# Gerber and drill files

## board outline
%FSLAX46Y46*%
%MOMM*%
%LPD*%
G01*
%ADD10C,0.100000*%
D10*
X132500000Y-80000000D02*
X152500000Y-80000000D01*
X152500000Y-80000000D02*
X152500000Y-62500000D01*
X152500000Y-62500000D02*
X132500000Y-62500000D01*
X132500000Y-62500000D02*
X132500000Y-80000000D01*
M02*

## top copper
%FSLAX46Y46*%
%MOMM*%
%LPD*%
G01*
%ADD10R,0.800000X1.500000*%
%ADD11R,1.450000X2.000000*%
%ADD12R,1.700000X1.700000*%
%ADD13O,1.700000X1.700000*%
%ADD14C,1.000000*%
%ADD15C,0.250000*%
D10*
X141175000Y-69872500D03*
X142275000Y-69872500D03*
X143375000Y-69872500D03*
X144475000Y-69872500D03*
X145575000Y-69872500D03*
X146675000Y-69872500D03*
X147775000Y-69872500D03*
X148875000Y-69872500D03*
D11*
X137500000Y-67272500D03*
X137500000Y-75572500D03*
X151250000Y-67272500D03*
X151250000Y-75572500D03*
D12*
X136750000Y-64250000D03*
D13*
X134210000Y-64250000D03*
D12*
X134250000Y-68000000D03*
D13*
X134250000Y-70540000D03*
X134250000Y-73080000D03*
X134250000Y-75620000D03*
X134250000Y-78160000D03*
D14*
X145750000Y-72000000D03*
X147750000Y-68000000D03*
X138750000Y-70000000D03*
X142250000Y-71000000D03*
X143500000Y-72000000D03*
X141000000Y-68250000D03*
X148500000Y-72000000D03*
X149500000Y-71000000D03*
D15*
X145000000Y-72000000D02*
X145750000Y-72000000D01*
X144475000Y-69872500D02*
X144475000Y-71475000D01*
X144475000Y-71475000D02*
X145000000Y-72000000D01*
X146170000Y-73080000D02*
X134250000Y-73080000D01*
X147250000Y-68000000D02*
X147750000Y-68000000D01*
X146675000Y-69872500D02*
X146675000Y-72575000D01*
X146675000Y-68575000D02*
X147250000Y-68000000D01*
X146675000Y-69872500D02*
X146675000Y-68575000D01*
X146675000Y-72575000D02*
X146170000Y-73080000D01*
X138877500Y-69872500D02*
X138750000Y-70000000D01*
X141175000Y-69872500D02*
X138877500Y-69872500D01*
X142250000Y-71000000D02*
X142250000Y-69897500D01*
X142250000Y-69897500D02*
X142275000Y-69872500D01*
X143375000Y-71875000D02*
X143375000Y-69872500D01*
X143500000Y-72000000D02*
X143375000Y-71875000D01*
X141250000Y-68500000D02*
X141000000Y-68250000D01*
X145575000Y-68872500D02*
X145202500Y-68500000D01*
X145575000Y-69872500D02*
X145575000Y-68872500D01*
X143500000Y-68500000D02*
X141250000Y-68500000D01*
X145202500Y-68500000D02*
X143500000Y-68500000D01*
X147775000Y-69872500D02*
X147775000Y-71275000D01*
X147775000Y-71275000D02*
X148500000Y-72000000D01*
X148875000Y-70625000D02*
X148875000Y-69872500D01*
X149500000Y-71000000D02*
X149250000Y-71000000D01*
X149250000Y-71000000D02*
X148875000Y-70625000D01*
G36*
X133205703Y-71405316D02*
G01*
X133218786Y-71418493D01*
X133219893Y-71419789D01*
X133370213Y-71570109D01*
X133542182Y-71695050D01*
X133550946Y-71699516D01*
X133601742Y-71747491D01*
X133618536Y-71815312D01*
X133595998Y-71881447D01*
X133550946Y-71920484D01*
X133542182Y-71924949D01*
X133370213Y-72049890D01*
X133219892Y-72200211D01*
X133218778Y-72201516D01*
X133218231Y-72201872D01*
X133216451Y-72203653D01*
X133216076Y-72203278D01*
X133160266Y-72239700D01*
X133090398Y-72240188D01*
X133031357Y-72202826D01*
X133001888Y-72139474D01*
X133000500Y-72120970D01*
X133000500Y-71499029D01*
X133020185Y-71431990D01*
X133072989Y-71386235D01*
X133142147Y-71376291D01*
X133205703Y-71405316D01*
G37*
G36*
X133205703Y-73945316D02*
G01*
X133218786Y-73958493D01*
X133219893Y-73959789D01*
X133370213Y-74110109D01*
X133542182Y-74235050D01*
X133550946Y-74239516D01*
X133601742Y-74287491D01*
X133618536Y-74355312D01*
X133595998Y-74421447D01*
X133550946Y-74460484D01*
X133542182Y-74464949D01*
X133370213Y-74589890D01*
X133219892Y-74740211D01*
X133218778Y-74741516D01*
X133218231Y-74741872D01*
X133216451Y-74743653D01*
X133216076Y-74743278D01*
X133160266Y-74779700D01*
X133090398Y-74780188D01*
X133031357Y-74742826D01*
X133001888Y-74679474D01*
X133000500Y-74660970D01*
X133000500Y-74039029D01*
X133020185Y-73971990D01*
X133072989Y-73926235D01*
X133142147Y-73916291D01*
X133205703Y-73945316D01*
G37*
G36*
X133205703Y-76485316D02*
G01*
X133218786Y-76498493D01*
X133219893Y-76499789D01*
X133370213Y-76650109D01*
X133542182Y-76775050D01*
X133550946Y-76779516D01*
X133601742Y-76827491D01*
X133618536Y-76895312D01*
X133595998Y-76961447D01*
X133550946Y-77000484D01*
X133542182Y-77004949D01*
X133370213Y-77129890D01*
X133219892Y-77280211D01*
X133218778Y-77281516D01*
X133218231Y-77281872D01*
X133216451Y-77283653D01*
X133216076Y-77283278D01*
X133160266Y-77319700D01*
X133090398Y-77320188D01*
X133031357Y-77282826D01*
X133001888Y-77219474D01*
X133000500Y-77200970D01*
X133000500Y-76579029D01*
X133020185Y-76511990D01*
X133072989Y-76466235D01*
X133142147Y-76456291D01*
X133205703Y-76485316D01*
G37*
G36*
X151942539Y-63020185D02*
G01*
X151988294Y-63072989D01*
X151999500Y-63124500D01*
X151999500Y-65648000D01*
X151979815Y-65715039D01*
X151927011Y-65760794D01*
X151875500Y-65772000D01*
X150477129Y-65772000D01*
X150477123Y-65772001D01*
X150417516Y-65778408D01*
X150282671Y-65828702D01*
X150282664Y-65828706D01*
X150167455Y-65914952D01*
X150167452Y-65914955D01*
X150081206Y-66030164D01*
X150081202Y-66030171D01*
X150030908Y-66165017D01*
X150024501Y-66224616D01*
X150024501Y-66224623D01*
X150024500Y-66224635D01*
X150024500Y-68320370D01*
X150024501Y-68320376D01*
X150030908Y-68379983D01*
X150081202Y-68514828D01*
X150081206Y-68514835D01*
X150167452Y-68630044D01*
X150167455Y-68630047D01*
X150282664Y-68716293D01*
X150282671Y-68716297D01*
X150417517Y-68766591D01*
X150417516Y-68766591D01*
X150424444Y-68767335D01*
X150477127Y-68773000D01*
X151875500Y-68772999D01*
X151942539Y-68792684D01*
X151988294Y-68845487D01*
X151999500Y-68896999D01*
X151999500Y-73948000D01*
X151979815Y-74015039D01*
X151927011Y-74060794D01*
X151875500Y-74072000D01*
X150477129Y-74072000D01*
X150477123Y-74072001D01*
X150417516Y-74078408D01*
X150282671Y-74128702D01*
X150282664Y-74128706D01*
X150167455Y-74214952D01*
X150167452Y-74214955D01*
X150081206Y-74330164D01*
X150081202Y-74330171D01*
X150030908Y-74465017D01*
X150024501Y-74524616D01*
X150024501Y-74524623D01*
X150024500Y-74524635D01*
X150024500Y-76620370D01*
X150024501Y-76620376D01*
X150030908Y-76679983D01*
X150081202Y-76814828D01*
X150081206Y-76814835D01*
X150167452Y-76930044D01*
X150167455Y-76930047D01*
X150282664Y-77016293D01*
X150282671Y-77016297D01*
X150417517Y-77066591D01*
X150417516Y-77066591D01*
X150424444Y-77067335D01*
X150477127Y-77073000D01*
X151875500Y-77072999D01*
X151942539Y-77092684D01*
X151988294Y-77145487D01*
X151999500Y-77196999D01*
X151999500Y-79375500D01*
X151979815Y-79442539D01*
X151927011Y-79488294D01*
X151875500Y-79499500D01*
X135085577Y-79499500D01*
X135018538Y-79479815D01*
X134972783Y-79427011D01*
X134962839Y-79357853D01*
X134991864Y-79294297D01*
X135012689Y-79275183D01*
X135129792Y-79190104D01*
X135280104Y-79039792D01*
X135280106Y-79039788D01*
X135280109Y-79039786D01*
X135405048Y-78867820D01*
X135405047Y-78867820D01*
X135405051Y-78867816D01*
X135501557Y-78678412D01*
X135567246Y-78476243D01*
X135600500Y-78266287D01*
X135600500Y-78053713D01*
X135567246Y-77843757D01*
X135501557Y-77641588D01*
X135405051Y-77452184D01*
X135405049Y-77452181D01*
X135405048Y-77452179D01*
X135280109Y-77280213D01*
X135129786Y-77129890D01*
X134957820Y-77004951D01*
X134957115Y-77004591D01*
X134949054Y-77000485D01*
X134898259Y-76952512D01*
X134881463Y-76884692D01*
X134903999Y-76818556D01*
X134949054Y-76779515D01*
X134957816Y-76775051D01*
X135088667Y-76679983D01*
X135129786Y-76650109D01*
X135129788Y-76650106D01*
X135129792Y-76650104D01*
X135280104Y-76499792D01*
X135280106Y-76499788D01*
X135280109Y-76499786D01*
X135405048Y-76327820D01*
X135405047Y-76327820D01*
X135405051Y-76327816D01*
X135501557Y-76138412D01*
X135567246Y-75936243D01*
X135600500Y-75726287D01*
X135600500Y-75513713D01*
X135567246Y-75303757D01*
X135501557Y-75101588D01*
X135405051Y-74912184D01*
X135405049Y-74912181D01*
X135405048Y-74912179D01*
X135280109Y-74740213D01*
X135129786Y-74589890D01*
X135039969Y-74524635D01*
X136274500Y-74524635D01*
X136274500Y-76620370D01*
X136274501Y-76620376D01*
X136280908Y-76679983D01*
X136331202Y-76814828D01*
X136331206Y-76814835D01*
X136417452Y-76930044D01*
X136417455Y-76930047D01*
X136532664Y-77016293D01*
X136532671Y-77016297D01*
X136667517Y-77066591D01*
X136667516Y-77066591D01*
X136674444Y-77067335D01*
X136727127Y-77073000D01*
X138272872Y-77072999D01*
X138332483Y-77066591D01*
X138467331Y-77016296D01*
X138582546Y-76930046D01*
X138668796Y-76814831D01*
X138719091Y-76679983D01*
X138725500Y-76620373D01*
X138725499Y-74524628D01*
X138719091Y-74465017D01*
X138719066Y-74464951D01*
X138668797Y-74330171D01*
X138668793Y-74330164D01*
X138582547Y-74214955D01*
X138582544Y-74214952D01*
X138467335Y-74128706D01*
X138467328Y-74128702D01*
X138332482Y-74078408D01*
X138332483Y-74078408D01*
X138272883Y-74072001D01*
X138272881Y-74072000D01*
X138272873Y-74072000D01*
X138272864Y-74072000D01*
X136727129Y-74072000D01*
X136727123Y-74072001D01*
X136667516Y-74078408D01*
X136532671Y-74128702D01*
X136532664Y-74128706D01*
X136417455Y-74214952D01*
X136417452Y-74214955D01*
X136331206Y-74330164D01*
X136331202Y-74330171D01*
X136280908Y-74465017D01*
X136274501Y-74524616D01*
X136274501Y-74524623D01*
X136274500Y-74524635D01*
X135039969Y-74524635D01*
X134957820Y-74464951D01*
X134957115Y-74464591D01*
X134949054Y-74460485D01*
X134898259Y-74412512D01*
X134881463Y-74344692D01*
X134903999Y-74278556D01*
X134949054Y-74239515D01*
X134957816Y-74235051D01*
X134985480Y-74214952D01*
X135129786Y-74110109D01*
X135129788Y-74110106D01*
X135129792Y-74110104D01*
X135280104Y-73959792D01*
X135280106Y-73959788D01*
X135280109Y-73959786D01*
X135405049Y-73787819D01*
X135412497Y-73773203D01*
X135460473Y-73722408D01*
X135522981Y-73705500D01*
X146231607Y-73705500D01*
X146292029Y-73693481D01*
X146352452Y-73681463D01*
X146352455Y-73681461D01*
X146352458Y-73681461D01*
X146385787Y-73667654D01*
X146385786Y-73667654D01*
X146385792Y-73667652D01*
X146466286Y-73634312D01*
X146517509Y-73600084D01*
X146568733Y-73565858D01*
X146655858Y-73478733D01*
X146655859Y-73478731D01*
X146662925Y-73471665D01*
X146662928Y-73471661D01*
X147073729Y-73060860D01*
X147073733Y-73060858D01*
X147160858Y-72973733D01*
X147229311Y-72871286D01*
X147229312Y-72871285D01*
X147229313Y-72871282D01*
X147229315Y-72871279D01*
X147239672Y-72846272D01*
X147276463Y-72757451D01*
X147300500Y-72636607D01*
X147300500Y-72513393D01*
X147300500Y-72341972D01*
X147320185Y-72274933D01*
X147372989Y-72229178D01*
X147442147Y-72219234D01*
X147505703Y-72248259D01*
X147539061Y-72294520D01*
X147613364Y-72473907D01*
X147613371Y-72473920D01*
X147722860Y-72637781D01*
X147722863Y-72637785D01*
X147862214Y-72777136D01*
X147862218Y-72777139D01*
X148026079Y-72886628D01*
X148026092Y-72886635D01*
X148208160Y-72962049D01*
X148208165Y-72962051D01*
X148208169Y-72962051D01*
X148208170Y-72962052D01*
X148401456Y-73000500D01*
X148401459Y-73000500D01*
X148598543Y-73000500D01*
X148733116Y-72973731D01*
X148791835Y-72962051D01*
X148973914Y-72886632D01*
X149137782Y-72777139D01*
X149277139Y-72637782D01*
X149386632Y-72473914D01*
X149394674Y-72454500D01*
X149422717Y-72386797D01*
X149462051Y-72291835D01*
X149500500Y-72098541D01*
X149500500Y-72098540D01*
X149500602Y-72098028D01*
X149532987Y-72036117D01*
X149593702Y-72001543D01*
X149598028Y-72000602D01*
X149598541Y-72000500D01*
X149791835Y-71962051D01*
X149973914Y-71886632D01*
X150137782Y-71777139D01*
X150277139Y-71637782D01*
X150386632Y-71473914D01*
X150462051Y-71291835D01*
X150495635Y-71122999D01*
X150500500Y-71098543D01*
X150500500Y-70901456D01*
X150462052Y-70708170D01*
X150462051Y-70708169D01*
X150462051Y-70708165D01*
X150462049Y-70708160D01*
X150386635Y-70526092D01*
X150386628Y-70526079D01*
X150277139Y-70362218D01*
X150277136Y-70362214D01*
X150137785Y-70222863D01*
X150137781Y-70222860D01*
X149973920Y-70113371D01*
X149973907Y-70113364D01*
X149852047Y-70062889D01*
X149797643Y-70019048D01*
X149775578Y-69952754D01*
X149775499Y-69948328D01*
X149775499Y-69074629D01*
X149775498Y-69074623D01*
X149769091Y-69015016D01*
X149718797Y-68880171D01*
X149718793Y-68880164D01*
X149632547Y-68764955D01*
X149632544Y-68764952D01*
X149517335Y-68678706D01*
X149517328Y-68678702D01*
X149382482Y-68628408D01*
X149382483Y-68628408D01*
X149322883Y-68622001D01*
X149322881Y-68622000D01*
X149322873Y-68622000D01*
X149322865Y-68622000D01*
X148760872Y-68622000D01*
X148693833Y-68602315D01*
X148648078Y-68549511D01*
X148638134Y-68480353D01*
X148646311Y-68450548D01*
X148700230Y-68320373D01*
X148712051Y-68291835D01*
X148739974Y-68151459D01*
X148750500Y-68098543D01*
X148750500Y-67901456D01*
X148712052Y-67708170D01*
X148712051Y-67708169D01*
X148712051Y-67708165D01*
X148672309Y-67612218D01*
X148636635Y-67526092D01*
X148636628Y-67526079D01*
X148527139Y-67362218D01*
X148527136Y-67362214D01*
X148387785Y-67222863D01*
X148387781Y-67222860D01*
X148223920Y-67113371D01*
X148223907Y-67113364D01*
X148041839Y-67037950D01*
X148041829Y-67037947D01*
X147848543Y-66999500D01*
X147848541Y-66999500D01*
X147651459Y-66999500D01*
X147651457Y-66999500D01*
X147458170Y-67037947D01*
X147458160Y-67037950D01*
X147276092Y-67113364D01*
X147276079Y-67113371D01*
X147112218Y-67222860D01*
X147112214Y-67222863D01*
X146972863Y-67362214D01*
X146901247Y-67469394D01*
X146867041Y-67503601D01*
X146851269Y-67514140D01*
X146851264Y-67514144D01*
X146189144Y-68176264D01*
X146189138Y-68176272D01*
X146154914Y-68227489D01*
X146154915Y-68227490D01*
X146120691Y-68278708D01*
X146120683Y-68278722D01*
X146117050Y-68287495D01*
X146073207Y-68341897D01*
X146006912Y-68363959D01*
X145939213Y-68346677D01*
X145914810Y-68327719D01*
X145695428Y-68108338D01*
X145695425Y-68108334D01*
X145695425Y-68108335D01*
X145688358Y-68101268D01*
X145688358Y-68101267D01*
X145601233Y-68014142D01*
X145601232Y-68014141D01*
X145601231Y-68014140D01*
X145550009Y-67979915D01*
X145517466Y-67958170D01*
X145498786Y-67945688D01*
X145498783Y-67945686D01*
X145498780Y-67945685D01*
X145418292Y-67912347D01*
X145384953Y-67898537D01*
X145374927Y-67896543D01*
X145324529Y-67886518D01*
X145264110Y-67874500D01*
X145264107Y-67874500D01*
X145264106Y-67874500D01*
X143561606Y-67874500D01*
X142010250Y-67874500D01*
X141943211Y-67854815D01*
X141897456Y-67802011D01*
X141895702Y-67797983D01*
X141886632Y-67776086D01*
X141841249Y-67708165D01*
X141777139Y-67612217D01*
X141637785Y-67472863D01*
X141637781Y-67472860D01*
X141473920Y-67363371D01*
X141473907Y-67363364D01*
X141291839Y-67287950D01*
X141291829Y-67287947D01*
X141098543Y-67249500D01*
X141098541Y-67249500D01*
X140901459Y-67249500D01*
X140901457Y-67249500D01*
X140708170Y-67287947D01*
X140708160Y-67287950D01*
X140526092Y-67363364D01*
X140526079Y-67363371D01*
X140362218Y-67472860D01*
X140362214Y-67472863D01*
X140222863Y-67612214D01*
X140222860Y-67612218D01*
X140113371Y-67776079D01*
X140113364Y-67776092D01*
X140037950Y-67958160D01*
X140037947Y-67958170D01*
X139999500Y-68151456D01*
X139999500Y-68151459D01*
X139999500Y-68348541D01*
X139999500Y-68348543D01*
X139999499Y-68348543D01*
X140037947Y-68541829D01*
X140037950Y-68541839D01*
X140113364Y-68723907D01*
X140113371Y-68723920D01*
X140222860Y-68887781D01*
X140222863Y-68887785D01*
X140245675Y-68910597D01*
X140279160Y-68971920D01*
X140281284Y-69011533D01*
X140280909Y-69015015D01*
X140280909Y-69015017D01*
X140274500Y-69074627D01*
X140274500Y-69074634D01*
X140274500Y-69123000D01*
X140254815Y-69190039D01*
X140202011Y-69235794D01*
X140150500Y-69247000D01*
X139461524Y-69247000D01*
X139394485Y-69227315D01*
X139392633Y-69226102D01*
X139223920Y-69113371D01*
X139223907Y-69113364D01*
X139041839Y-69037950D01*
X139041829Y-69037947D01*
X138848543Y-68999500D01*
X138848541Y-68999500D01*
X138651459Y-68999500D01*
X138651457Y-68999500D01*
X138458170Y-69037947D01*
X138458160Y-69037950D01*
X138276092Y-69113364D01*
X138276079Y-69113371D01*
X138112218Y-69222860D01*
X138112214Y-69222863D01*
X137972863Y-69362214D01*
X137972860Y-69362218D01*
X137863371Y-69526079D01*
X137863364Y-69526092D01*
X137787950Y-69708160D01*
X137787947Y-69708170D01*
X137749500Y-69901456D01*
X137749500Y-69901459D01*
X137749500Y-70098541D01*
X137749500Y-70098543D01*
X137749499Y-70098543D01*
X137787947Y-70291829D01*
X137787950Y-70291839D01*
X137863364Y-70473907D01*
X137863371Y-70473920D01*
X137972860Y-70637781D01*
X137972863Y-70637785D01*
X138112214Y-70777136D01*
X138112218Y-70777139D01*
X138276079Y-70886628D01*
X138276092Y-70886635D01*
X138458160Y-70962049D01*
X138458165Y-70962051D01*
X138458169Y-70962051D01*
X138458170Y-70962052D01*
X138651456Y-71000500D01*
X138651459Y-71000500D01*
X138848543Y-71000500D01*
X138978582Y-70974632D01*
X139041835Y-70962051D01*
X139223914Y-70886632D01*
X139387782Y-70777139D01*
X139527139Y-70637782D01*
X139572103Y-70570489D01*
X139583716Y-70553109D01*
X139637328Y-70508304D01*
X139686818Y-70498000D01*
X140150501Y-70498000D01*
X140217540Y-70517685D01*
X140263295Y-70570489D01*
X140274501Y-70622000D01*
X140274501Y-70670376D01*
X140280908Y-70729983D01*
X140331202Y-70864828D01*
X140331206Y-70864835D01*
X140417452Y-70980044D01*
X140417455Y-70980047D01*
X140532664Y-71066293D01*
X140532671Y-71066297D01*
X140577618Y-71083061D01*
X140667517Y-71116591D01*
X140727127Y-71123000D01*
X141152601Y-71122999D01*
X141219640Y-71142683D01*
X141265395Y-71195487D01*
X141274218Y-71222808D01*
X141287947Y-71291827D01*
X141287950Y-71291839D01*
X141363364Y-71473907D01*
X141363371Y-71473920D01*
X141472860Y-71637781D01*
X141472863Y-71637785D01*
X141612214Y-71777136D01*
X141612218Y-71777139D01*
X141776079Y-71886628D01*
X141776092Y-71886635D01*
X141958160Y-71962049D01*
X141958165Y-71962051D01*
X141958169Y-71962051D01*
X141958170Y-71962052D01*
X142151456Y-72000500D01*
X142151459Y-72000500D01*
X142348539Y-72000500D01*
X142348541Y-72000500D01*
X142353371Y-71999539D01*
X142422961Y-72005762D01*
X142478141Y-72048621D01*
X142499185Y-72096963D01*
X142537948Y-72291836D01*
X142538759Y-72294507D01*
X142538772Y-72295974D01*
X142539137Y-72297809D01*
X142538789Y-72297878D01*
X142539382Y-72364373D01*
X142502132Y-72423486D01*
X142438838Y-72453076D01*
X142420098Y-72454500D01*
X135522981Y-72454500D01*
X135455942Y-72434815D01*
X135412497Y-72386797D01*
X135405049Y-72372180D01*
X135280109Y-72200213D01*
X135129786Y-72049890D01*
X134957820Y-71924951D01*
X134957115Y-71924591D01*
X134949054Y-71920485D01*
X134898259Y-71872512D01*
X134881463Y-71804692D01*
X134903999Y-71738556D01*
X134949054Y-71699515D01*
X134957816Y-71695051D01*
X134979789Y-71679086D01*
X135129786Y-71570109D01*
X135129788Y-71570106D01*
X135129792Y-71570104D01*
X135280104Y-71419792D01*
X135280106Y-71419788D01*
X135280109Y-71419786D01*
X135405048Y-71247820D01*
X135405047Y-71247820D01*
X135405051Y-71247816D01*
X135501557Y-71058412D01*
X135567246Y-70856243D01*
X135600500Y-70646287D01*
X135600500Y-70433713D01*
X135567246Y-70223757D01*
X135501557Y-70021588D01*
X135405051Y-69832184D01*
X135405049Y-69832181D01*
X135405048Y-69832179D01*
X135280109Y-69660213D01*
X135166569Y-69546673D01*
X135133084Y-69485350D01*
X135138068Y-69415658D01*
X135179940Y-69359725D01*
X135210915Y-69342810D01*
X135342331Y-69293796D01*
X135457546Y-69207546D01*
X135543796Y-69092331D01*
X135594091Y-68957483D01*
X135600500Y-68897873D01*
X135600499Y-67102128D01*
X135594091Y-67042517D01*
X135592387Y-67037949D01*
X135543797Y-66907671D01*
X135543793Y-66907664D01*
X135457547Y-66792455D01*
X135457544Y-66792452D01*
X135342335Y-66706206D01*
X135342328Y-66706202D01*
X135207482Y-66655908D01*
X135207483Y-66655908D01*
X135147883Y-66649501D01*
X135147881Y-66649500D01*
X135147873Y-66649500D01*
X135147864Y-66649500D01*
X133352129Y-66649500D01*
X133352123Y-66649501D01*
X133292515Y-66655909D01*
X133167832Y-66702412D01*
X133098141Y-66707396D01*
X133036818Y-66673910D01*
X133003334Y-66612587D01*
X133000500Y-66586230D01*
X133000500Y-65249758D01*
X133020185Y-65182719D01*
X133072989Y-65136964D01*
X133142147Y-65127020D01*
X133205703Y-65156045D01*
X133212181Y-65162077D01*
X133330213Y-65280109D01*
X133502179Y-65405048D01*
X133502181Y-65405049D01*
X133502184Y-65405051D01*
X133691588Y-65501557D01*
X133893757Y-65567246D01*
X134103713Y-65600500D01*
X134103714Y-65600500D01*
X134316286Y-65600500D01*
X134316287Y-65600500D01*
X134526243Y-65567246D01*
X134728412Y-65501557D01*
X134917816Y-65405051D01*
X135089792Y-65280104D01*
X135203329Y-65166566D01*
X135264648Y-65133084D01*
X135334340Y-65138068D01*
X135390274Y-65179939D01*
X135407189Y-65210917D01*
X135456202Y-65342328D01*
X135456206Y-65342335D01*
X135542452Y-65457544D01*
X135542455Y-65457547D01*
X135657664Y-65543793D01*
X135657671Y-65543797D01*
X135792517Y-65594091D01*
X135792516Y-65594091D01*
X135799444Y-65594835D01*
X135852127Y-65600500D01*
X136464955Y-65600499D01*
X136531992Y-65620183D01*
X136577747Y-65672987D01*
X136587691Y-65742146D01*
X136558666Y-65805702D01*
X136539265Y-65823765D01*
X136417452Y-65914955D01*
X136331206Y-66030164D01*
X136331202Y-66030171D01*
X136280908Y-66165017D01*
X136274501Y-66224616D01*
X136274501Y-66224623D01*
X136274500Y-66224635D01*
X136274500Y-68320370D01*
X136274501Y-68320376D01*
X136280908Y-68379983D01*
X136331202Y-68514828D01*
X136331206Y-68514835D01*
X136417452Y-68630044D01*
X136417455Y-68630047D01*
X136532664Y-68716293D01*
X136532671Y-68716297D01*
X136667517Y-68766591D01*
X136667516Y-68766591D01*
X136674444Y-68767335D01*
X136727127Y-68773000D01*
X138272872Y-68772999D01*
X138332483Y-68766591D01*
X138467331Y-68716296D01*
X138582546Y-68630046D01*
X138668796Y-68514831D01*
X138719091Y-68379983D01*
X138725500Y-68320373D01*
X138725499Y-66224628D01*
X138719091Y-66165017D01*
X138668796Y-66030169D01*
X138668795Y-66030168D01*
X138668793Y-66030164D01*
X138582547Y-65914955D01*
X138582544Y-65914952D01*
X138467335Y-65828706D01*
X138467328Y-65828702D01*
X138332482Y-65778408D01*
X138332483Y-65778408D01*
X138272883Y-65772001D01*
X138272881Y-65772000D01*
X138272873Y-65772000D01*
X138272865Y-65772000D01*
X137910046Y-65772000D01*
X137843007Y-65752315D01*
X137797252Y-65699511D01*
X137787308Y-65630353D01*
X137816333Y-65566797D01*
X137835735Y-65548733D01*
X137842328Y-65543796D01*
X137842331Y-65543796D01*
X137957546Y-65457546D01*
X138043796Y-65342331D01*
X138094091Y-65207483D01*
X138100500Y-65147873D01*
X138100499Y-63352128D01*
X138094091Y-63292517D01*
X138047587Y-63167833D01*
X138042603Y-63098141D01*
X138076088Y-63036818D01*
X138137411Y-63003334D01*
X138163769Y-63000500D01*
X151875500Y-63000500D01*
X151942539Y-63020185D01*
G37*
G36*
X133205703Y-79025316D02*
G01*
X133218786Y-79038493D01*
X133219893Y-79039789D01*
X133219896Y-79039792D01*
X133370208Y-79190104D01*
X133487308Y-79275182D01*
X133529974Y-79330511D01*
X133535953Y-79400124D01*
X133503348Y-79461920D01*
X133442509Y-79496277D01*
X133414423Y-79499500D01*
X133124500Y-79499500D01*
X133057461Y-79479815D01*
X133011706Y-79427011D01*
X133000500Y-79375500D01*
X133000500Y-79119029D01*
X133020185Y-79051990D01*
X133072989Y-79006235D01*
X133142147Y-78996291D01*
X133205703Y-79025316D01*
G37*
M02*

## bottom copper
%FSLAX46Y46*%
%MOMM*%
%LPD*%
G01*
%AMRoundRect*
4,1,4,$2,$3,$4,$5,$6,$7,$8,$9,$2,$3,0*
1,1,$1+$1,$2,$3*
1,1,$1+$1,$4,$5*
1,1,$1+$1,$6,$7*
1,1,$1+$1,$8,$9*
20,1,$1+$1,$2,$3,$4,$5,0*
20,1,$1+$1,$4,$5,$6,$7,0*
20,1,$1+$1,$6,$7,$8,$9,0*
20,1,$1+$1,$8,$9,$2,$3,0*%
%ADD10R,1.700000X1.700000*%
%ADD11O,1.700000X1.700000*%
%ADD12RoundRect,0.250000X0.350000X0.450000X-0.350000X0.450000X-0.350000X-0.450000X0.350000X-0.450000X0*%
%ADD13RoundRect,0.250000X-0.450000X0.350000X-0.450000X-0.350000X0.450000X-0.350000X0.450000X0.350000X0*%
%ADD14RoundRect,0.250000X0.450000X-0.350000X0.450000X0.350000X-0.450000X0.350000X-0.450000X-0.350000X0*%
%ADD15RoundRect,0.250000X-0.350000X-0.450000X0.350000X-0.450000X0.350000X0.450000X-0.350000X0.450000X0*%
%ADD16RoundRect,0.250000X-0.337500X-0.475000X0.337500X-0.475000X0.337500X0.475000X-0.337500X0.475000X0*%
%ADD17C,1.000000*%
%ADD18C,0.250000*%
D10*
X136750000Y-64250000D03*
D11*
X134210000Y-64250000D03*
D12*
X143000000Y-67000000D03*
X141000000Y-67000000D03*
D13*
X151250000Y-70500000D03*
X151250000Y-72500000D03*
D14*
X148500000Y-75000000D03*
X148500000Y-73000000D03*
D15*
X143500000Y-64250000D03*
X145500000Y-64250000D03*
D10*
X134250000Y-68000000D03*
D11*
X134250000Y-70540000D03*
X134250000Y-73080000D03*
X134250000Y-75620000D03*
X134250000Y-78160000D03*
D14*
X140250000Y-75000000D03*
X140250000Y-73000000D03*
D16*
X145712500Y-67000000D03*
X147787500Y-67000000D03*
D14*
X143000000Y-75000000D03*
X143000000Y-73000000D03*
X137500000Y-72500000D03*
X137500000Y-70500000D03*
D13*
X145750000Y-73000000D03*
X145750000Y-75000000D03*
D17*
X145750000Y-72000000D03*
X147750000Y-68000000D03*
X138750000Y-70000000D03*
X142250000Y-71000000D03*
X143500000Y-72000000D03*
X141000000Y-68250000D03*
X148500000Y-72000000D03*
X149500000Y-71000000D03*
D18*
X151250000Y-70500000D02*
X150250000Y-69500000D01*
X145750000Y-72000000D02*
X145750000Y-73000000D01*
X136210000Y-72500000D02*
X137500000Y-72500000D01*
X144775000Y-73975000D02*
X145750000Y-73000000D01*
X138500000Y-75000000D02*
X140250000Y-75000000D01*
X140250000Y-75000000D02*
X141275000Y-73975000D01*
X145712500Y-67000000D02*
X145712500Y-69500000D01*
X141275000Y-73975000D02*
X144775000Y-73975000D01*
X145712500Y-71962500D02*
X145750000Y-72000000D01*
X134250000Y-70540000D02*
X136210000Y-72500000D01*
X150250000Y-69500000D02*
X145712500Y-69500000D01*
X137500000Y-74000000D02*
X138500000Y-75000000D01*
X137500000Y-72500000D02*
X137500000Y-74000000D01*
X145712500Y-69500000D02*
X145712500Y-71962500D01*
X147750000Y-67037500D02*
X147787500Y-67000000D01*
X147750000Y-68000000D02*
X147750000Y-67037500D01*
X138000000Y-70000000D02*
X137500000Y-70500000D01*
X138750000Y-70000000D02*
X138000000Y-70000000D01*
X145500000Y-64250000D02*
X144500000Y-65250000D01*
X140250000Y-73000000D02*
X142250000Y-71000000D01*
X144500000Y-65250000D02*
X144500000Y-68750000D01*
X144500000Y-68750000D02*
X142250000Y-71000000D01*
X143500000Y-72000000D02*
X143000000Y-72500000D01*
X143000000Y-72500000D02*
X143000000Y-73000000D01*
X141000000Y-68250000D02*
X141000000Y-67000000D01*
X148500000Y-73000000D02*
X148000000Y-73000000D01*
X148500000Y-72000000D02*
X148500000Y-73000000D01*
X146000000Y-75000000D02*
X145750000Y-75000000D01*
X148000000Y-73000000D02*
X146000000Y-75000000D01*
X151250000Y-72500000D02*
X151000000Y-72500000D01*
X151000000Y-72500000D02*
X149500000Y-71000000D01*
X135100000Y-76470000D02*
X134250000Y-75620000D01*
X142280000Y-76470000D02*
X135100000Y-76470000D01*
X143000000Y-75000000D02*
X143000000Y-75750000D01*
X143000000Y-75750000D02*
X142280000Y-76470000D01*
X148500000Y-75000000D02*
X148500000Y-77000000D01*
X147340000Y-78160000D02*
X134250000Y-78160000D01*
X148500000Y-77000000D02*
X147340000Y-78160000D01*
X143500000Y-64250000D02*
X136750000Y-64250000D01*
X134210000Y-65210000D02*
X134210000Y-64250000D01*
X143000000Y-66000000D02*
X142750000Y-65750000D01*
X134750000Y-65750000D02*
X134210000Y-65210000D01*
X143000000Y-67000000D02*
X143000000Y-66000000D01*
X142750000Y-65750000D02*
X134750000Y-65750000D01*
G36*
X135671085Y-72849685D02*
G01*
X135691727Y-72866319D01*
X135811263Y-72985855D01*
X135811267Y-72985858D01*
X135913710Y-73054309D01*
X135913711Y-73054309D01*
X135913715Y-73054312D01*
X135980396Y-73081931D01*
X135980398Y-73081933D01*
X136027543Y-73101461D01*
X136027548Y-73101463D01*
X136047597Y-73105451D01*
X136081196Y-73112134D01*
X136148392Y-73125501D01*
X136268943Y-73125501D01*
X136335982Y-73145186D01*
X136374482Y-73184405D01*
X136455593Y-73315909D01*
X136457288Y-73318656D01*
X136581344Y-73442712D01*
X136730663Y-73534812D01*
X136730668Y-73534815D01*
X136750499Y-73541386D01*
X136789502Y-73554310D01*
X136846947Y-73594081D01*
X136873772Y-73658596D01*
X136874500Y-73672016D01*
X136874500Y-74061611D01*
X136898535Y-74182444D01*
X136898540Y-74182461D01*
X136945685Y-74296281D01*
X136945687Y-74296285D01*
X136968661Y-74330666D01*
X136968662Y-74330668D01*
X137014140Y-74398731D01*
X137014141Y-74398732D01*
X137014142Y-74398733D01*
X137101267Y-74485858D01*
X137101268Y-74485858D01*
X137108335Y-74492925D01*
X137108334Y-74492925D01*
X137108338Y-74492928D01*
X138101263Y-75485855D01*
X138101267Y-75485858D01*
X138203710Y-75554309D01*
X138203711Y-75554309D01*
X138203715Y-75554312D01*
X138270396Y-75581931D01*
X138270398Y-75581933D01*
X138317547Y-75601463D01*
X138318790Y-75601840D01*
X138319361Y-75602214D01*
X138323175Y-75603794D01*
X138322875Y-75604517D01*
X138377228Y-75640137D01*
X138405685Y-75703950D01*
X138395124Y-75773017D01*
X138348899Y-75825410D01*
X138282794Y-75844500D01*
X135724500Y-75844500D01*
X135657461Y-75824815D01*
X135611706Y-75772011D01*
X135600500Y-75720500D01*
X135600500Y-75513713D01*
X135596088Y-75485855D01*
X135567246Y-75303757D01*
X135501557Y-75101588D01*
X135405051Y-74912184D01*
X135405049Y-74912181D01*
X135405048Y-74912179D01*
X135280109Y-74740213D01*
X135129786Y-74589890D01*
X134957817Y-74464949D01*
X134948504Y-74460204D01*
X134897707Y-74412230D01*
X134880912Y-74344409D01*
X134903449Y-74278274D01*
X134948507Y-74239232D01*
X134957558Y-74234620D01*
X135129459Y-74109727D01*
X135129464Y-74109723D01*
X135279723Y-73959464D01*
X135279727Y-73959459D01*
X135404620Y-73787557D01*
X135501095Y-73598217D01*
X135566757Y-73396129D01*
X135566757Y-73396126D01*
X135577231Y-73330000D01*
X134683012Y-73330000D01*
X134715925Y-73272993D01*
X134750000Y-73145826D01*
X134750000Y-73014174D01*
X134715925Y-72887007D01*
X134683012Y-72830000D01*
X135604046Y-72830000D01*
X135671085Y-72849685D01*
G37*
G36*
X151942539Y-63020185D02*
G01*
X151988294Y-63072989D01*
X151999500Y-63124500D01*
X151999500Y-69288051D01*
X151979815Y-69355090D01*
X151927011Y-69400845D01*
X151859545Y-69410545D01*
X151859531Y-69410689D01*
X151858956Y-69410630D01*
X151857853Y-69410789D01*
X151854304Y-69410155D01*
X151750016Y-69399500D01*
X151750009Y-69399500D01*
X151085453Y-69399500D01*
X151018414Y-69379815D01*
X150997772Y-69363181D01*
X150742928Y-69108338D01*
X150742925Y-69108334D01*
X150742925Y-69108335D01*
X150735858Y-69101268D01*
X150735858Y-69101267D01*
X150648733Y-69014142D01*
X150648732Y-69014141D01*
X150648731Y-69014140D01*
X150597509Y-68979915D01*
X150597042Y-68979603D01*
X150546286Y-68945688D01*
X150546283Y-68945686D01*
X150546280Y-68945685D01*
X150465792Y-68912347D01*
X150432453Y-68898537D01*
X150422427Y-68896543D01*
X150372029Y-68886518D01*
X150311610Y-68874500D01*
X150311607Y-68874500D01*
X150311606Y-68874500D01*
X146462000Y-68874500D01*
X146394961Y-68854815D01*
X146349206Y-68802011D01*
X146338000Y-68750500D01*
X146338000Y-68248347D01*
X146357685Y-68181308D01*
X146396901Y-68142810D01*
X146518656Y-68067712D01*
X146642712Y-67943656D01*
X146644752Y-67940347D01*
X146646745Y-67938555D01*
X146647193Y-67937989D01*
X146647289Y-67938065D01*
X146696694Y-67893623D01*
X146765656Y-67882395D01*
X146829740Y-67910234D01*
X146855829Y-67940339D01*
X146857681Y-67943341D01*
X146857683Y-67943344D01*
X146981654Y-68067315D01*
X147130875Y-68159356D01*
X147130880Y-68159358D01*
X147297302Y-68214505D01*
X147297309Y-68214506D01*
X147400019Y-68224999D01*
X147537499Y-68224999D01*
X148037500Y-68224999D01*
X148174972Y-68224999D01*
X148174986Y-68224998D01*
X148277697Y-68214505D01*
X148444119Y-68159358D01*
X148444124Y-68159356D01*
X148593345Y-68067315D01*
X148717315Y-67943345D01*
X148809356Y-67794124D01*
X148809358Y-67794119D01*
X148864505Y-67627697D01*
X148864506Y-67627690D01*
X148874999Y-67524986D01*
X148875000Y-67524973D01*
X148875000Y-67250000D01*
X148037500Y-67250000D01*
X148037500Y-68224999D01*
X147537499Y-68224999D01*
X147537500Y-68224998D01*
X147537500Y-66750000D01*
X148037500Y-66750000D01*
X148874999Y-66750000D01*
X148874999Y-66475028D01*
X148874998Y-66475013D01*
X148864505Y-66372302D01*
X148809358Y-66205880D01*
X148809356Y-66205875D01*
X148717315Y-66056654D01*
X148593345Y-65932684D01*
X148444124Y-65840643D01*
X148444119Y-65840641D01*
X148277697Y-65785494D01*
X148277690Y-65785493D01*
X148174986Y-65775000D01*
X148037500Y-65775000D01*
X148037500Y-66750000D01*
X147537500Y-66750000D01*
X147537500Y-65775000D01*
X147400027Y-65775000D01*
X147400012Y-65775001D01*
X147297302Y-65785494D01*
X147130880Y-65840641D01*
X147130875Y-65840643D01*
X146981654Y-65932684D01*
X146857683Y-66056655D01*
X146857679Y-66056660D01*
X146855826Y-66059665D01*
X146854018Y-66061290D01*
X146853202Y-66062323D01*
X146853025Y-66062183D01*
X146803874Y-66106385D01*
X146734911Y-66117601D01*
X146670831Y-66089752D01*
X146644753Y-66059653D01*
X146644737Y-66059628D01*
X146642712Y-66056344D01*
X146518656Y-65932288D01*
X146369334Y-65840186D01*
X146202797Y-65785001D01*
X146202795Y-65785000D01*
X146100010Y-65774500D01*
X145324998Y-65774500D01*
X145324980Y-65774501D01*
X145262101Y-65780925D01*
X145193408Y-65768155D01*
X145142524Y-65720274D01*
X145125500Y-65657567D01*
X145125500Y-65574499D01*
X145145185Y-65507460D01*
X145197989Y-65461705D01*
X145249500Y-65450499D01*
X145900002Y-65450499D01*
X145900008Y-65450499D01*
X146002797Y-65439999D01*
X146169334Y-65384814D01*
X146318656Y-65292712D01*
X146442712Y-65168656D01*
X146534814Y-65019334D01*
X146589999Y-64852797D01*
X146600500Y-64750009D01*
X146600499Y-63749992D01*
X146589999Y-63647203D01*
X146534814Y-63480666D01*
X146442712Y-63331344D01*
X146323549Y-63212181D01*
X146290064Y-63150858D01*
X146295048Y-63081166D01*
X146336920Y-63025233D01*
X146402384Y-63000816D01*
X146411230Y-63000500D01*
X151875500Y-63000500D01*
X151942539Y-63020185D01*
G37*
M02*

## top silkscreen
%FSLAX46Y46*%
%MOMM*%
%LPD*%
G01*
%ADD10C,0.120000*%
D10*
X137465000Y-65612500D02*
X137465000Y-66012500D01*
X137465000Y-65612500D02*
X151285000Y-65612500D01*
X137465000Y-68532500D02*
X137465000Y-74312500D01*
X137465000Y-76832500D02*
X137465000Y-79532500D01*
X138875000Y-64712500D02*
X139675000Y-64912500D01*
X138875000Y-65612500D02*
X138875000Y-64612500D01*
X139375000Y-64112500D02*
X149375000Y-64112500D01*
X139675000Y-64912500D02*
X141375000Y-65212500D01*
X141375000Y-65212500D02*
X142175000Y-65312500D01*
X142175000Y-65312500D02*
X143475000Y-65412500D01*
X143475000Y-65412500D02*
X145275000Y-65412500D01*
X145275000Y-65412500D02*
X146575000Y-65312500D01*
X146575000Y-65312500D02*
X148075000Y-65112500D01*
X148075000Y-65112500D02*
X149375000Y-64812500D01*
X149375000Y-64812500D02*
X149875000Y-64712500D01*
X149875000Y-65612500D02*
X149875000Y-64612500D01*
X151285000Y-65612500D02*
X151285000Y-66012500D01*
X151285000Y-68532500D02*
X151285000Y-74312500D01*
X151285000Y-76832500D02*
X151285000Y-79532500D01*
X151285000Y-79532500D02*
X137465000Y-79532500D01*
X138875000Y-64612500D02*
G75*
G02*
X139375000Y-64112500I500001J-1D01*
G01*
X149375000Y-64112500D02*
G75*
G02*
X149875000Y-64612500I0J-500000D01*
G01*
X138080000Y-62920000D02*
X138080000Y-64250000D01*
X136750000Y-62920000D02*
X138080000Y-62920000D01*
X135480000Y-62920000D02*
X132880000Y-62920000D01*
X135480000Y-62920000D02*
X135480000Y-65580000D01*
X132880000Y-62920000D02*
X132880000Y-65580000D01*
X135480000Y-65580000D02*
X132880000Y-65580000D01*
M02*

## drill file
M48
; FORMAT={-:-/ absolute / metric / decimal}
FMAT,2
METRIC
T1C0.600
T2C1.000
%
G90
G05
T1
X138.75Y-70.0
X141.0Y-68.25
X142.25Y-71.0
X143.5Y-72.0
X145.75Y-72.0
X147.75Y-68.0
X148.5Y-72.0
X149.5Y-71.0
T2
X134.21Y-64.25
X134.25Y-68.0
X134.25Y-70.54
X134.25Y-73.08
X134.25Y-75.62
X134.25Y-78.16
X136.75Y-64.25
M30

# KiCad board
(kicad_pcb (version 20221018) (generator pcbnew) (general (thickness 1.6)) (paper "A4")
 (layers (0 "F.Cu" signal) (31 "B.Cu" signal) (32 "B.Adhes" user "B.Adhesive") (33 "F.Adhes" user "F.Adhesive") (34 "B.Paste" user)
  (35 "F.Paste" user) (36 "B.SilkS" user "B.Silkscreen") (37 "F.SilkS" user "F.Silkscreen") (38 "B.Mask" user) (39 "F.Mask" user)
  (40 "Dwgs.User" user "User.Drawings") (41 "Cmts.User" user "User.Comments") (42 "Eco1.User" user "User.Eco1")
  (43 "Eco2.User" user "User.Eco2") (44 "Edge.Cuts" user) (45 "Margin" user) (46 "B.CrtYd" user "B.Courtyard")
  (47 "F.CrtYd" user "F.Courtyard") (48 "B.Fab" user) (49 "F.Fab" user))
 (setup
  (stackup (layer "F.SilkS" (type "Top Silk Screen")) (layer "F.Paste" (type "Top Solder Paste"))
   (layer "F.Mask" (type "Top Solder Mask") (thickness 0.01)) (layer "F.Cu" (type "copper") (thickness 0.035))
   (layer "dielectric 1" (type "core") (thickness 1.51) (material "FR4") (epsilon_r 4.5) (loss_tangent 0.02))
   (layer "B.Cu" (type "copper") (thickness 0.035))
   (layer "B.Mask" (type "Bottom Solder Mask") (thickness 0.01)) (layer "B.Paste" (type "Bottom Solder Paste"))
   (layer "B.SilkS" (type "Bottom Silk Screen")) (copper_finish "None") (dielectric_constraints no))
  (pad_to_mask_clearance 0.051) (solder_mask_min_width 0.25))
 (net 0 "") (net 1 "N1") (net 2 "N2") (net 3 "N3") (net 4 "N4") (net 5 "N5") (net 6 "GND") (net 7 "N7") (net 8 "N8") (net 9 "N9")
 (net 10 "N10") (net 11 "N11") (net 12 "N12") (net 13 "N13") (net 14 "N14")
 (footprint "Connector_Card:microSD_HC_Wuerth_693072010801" (layer "F.Cu") (at 144.375 71.4225)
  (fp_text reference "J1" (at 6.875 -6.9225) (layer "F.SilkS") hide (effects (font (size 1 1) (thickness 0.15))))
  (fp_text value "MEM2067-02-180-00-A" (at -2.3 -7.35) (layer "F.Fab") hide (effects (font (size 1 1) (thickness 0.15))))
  (fp_line (start -6.91 -5.81) (end -6.91 -5.41) (stroke (width 0.12) (type solid)) (layer "F.SilkS"))
  (fp_line (start -6.91 -5.81) (end 6.91 -5.81) (stroke (width 0.12) (type solid)) (layer "F.SilkS"))
  (fp_line (start -6.91 -2.89) (end -6.91 2.89) (stroke (width 0.12) (type solid)) (layer "F.SilkS"))
  (fp_line (start -6.91 5.41) (end -6.91 8.11) (stroke (width 0.12) (type solid)) (layer "F.SilkS"))
  (fp_line (start -5.5 -6.71) (end -4.7 -6.51) (stroke (width 0.12) (type solid)) (layer "F.SilkS"))
  (fp_line (start -5.5 -5.81) (end -5.5 -6.81) (stroke (width 0.12) (type solid)) (layer "F.SilkS"))
  (fp_line (start -5 -7.31) (end 5 -7.31) (stroke (width 0.12) (type solid)) (layer "F.SilkS"))
  (fp_line (start -4.7 -6.51) (end -3 -6.21) (stroke (width 0.12) (type solid)) (layer "F.SilkS"))
  (fp_line (start -3 -6.21) (end -2.2 -6.11) (stroke (width 0.12) (type solid)) (layer "F.SilkS"))
  (fp_line (start -2.2 -6.11) (end -0.9 -6.01) (stroke (width 0.12) (type solid)) (layer "F.SilkS"))
  (fp_line (start -0.9 -6.01) (end 0.9 -6.01) (stroke (width 0.12) (type solid)) (layer "F.SilkS"))
  (fp_line (start 0.9 -6.01) (end 2.2 -6.11) (stroke (width 0.12) (type solid)) (layer "F.SilkS"))
  (fp_line (start 2.2 -6.11) (end 3.7 -6.31) (stroke (width 0.12) (type solid)) (layer "F.SilkS"))
  (fp_line (start 3.7 -6.31) (end 5 -6.61) (stroke (width 0.12) (type solid)) (layer "F.SilkS"))
  (fp_line (start 5 -6.61) (end 5.5 -6.71) (stroke (width 0.12) (type solid)) (layer "F.SilkS"))
  (fp_line (start 5.5 -5.81) (end 5.5 -6.81) (stroke (width 0.12) (type solid)) (layer "F.SilkS"))
  (fp_line (start 6.91 -5.81) (end 6.91 -5.41) (stroke (width 0.12) (type solid)) (layer "F.SilkS"))
  (fp_line (start 6.91 -2.89) (end 6.91 2.89) (stroke (width 0.12) (type solid)) (layer "F.SilkS"))
  (fp_line (start 6.91 5.41) (end 6.91 8.11) (stroke (width 0.12) (type solid)) (layer "F.SilkS"))
  (fp_line (start 6.91 8.11) (end -6.91 8.11) (stroke (width 0.12) (type solid)) (layer "F.SilkS"))
  (fp_arc (start -5.5 -6.81) (mid -5.353553 -7.163553) (end -5 -7.31) (stroke (width 0.12) (type solid)) (layer "F.SilkS"))
  (fp_arc (start 5 -7.31) (mid 5.353553 -7.163553) (end 5.5 -6.81) (stroke (width 0.12) (type solid)) (layer "F.SilkS"))
  (pad "1" smd rect (at -3.2 -1.55) (size 0.8 1.5) (layers "F.Cu" "F.Paste" "F.Mask") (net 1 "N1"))
  (pad "2" smd rect (at -2.1 -1.55) (size 0.8 1.5) (layers "F.Cu" "F.Paste" "F.Mask") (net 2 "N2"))
  (pad "3" smd rect (at -1 -1.55) (size 0.8 1.5) (layers "F.Cu" "F.Paste" "F.Mask") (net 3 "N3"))
  (pad "4" smd rect (at 0.1 -1.55) (size 0.8 1.5) (layers "F.Cu" "F.Paste" "F.Mask") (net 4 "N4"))
  (pad "5" smd rect (at 1.2 -1.55) (size 0.8 1.5) (layers "F.Cu" "F.Paste" "F.Mask") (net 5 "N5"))
  (pad "6" smd rect (at 2.3 -1.55) (size 0.8 1.5) (layers "F.Cu" "F.Paste" "F.Mask") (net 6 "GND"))
  (pad "7" smd rect (at 3.4 -1.55) (size 0.8 1.5) (layers "F.Cu" "F.Paste" "F.Mask") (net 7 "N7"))
  (pad "8" smd rect (at 4.5 -1.55) (size 0.8 1.5) (layers "F.Cu" "F.Paste" "F.Mask") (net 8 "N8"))
  (pad "9" smd rect (at -6.875 -4.15) (size 1.45 2) (layers "F.Cu" "F.Paste" "F.Mask") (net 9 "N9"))
  (pad "9" smd rect (at -6.875 4.15) (size 1.45 2) (layers "F.Cu" "F.Paste" "F.Mask") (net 9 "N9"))
  (pad "9" smd rect (at 6.875 -4.15) (size 1.45 2) (layers "F.Cu" "F.Paste" "F.Mask") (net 9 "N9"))
  (pad "9" smd rect (at 6.875 4.15) (size 1.45 2) (layers "F.Cu" "F.Paste" "F.Mask") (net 9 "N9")))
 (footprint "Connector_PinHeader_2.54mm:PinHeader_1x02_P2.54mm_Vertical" (layer "F.Cu") (at 136.75 64.25 -90)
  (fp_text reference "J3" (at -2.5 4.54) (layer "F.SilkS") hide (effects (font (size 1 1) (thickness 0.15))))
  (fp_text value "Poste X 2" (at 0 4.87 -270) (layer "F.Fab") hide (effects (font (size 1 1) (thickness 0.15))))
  (fp_line (start -1.33 -1.33) (end 0 -1.33) (stroke (width 0.12) (type solid)) (layer "F.SilkS"))
  (fp_line (start -1.33 0) (end -1.33 -1.33) (stroke (width 0.12) (type solid)) (layer "F.SilkS"))
  (fp_line (start -1.33 1.27) (end -1.33 3.87) (stroke (width 0.12) (type solid)) (layer "F.SilkS"))
  (fp_line (start -1.33 1.27) (end 1.33 1.27) (stroke (width 0.12) (type solid)) (layer "F.SilkS"))
  (fp_line (start -1.33 3.87) (end 1.33 3.87) (stroke (width 0.12) (type solid)) (layer "F.SilkS"))
  (fp_line (start 1.33 1.27) (end 1.33 3.87) (stroke (width 0.12) (type solid)) (layer "F.SilkS"))
  (pad "1" thru_hole rect (at 0 0 270) (size 1.7 1.7) (drill 1) (layers "*.Cu" "*.Mask") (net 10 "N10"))
  (pad "2" thru_hole oval (at 0 2.54 270) (size 1.7 1.7) (drill 1) (layers "*.Cu" "*.Mask") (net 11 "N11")))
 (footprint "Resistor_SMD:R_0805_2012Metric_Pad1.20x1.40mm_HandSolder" (layer "B.Cu") (at 142 67 180)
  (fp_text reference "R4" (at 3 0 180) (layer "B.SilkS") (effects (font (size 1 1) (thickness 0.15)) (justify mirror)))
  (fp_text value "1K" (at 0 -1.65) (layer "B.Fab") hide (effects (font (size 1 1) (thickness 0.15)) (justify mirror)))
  (pad "1" smd roundrect (at -1 0 180) (size 1.2 1.4) (layers "B.Cu" "B.Paste" "B.Mask") (roundrect_rratio 0.2083333333) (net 11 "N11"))
  (pad "2" smd roundrect (at 1 0 180) (size 1.2 1.4) (layers "B.Cu" "B.Paste" "B.Mask") (roundrect_rratio 0.2083333333) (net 5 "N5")))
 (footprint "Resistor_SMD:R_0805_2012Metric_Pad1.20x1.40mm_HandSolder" (layer "B.Cu") (at 151.25 71.5 -90)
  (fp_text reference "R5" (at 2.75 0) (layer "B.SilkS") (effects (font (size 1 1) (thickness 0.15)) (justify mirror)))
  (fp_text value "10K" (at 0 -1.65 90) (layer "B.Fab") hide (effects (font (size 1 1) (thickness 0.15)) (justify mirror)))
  (pad "1" smd roundrect (at -1 0 270) (size 1.2 1.4) (layers "B.Cu" "B.Paste" "B.Mask") (roundrect_rratio 0.2083333333) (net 4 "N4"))
  (pad "2" smd roundrect (at 1 0 270) (size 1.2 1.4) (layers "B.Cu" "B.Paste" "B.Mask") (roundrect_rratio 0.2083333333) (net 8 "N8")))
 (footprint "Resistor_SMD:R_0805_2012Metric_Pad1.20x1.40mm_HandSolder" (layer "B.Cu") (at 148.5 74 90)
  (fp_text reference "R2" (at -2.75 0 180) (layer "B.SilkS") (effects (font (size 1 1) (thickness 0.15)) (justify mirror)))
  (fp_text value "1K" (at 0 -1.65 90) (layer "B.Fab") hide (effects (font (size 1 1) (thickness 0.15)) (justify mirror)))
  (pad "1" smd roundrect (at -1 0 90) (size 1.2 1.4) (layers "B.Cu" "B.Paste" "B.Mask") (roundrect_rratio 0.2083333333) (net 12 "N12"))
  (pad "2" smd roundrect (at 1 0 90) (size 1.2 1.4) (layers "B.Cu" "B.Paste" "B.Mask") (roundrect_rratio 0.2083333333) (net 7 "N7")))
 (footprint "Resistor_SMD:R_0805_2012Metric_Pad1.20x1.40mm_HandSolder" (layer "B.Cu") (at 144.5 64.25)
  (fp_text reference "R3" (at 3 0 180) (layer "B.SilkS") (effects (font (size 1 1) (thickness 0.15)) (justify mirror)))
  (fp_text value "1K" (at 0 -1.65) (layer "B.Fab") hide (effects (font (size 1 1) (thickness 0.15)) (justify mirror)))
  (pad "1" smd roundrect (at -1 0) (size 1.2 1.4) (layers "B.Cu" "B.Paste" "B.Mask") (roundrect_rratio 0.2083333333) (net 10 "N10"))
  (pad "2" smd roundrect (at 1 0) (size 1.2 1.4) (layers "B.Cu" "B.Paste" "B.Mask") (roundrect_rratio 0.2083333333) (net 2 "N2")))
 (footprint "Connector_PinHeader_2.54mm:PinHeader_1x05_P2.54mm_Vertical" (layer "B.Cu") (at 134.25 68 180)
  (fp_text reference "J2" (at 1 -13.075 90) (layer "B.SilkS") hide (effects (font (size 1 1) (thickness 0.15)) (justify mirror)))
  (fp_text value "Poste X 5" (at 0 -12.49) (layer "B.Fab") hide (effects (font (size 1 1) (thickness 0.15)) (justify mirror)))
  (pad "1" thru_hole rect (at 0 0 180) (size 1.7 1.7) (drill 1) (layers "*.Cu" "*.Mask") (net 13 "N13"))
  (pad "2" thru_hole oval (at 0 -2.54 180) (size 1.7 1.7) (drill 1) (layers "*.Cu" "*.Mask") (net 4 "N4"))
  (pad "3" thru_hole oval (at 0 -5.08 180) (size 1.7 1.7) (drill 1) (layers "*.Cu" "*.Mask") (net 6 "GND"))
  (pad "4" thru_hole oval (at 0 -7.62 180) (size 1.7 1.7) (drill 1) (layers "*.Cu" "*.Mask") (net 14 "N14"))
  (pad "5" thru_hole oval (at 0 -10.16 180) (size 1.7 1.7) (drill 1) (layers "*.Cu" "*.Mask") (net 12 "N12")))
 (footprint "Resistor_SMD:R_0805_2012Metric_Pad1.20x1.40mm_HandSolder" (layer "B.Cu") (at 140.25 74 90)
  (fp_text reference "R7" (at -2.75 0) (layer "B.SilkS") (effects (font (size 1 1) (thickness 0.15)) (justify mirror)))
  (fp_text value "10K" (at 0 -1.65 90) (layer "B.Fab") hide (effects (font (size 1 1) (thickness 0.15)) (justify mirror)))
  (pad "1" smd roundrect (at -1 0 90) (size 1.2 1.4) (layers "B.Cu" "B.Paste" "B.Mask") (roundrect_rratio 0.2083333333) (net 4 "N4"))
  (pad "2" smd roundrect (at 1 0 90) (size 1.2 1.4) (layers "B.Cu" "B.Paste" "B.Mask") (roundrect_rratio 0.2083333333) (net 2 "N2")))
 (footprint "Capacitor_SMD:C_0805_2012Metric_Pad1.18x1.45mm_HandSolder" (layer "B.Cu") (at 146.75 67)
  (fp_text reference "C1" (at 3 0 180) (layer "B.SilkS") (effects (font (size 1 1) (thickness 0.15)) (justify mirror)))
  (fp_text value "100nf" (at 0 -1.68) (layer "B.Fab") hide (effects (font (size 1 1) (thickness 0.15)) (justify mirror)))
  (pad "1" smd roundrect (at -1.0375 0) (size 1.175 1.45) (layers "B.Cu" "B.Paste" "B.Mask") (roundrect_rratio 0.2127659574) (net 4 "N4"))
  (pad "2" smd roundrect (at 1.0375 0) (size 1.175 1.45) (layers "B.Cu" "B.Paste" "B.Mask") (roundrect_rratio 0.2127659574) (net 6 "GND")))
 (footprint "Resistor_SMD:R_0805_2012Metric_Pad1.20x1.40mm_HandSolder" (layer "B.Cu") (at 143 74 90)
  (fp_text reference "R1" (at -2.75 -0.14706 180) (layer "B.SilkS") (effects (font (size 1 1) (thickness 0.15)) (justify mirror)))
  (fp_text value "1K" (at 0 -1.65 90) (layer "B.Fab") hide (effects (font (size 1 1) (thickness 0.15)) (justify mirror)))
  (pad "1" smd roundrect (at -1 0 90) (size 1.2 1.4) (layers "B.Cu" "B.Paste" "B.Mask") (roundrect_rratio 0.2083333333) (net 14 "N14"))
  (pad "2" smd roundrect (at 1 0 90) (size 1.2 1.4) (layers "B.Cu" "B.Paste" "B.Mask") (roundrect_rratio 0.2083333333) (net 3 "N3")))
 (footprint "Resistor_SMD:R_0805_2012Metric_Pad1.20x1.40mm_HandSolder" (layer "B.Cu") (at 137.5 71.5 90)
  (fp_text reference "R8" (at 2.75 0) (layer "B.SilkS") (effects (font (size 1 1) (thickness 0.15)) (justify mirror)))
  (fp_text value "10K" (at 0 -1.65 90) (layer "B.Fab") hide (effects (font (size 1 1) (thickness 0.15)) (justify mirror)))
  (pad "1" smd roundrect (at -1 0 90) (size 1.2 1.4) (layers "B.Cu" "B.Paste" "B.Mask") (roundrect_rratio 0.2083333333) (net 4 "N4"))
  (pad "2" smd roundrect (at 1 0 90) (size 1.2 1.4) (layers "B.Cu" "B.Paste" "B.Mask") (roundrect_rratio 0.2083333333) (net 1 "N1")))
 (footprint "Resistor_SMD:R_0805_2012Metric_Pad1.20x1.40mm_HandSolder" (layer "B.Cu") (at 145.75 74 -90)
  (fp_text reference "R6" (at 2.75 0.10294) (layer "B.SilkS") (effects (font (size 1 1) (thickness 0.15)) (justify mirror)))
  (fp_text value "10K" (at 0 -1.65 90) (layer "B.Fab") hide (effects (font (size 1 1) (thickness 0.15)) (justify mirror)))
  (pad "1" smd roundrect (at -1 0 270) (size 1.2 1.4) (layers "B.Cu" "B.Paste" "B.Mask") (roundrect_rratio 0.2083333333) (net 4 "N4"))
  (pad "2" smd roundrect (at 1 0 270) (size 1.2 1.4) (layers "B.Cu" "B.Paste" "B.Mask") (roundrect_rratio 0.2083333333) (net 7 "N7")))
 (gr_line (start 132.5 80) (end 152.5 80) (stroke (width 0.1) (type default)) (layer "Edge.Cuts"))
 (gr_line (start 152.5 80) (end 152.5 62.5) (stroke (width 0.1) (type default)) (layer "Edge.Cuts"))
 (gr_line (start 152.5 62.5) (end 132.5 62.5) (stroke (width 0.1) (type default)) (layer "Edge.Cuts"))
 (gr_line (start 132.5 62.5) (end 132.5 80) (stroke (width 0.1) (type default)) (layer "Edge.Cuts"))
 (segment (start 145 72) (end 145.75 72) (width 0.25) (layer "F.Cu") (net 4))
 (segment (start 144.475 69.8725) (end 144.475 71.475) (width 0.25) (layer "F.Cu") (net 4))
 (segment (start 144.475 71.475) (end 145 72) (width 0.25) (layer "F.Cu") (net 4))
 (via (at 145.75 72) (size 1) (drill 0.6) (layers "F.Cu" "B.Cu") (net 4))
 (segment (start 151.25 70.5) (end 150.25 69.5) (width 0.25) (layer "B.Cu") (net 4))
 (segment (start 145.75 72) (end 145.75 73) (width 0.25) (layer "B.Cu") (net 4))
 (segment (start 136.21 72.5) (end 137.5 72.5) (width 0.25) (layer "B.Cu") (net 4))
 (segment (start 144.775 73.975) (end 145.75 73) (width 0.25) (layer "B.Cu") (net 4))
 (segment (start 138.5 75) (end 140.25 75) (width 0.25) (layer "B.Cu") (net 4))
 (segment (start 140.25 75) (end 141.275 73.975) (width 0.25) (layer "B.Cu") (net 4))
 (segment (start 145.7125 67) (end 145.7125 69.5) (width 0.25) (layer "B.Cu") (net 4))
 (segment (start 141.275 73.975) (end 144.775 73.975) (width 0.25) (layer "B.Cu") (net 4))
 (segment (start 145.7125 71.9625) (end 145.75 72) (width 0.25) (layer "B.Cu") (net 4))
 (segment (start 134.25 70.54) (end 136.21 72.5) (width 0.25) (layer "B.Cu") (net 4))
 (segment (start 150.25 69.5) (end 145.7125 69.5) (width 0.25) (layer "B.Cu") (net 4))
 (segment (start 137.5 74) (end 138.5 75) (width 0.25) (layer "B.Cu") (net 4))
 (segment (start 137.5 72.5) (end 137.5 74) (width 0.25) (layer "B.Cu") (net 4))
 (segment (start 145.7125 69.5) (end 145.7125 71.9625) (width 0.25) (layer "B.Cu") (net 4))
 (segment (start 146.17 73.08) (end 134.25 73.08) (width 0.25) (layer "F.Cu") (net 6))
 (segment (start 147.25 68) (end 147.75 68) (width 0.25) (layer "F.Cu") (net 6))
 (segment (start 146.675 69.8725) (end 146.675 72.575) (width 0.25) (layer "F.Cu") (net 6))
 (segment (start 146.675 68.575) (end 147.25 68) (width 0.25) (layer "F.Cu") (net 6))
 (segment (start 146.675 69.8725) (end 146.675 68.575) (width 0.25) (layer "F.Cu") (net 6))
 (segment (start 146.675 72.575) (end 146.17 73.08) (width 0.25) (layer "F.Cu") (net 6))
 (via (at 147.75 68) (size 1) (drill 0.6) (layers "F.Cu" "B.Cu") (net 6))
 (segment (start 147.75 67.0375) (end 147.7875 67) (width 0.25) (layer "B.Cu") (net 6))
 (segment (start 147.75 68) (end 147.75 67.0375) (width 0.25) (layer "B.Cu") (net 6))
 (segment (start 138.8775 69.8725) (end 138.75 70) (width 0.25) (layer "F.Cu") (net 1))
 (segment (start 141.175 69.8725) (end 138.8775 69.8725) (width 0.25) (layer "F.Cu") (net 1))
 (via (at 138.75 70) (size 1) (drill 0.6) (layers "F.Cu" "B.Cu") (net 1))
 (segment (start 138 70) (end 137.5 70.5) (width 0.25) (layer "B.Cu") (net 1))
 (segment (start 138.75 70) (end 138 70) (width 0.25) (layer "B.Cu") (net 1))
 (segment (start 142.25 71) (end 142.25 69.8975) (width 0.25) (layer "F.Cu") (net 2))
 (segment (start 142.25 69.8975) (end 142.275 69.8725) (width 0.25) (layer "F.Cu") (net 2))
 (via (at 142.25 71) (size 1) (drill 0.6) (layers "F.Cu" "B.Cu") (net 2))
 (segment (start 145.5 64.25) (end 144.5 65.25) (width 0.25) (layer "B.Cu") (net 2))
 (segment (start 140.25 73) (end 142.25 71) (width 0.25) (layer "B.Cu") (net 2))
 (segment (start 144.5 65.25) (end 144.5 68.75) (width 0.25) (layer "B.Cu") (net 2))
 (segment (start 144.5 68.75) (end 142.25 71) (width 0.25) (layer "B.Cu") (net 2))
 (segment (start 143.375 71.875) (end 143.375 69.8725) (width 0.25) (layer "F.Cu") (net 3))
 (segment (start 143.5 72) (end 143.375 71.875) (width 0.25) (layer "F.Cu") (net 3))
 (via (at 143.5 72) (size 1) (drill 0.6) (layers "F.Cu" "B.Cu") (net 3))
 (segment (start 143.5 72) (end 143 72.5) (width 0.25) (layer "B.Cu") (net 3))
 (segment (start 143 72.5) (end 143 73) (width 0.25) (layer "B.Cu") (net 3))
 (segment (start 141.25 68.5) (end 141 68.25) (width 0.25) (layer "F.Cu") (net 5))
 (segment (start 145.575 68.8725) (end 145.2025 68.5) (width 0.25) (layer "F.Cu") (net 5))
 (segment (start 145.575 69.8725) (end 145.575 68.8725) (width 0.25) (layer "F.Cu") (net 5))
 (segment (start 143.5 68.5) (end 141.25 68.5) (width 0.25) (layer "F.Cu") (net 5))
 (segment (start 145.2025 68.5) (end 143.5 68.5) (width 0.25) (layer "F.Cu") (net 5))
 (via (at 141 68.25) (size 1) (drill 0.6) (layers "F.Cu" "B.Cu") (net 5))
 (segment (start 141 68.25) (end 141 67) (width 0.25) (layer "B.Cu") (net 5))
 (segment (start 147.775 69.8725) (end 147.775 71.275) (width 0.25) (layer "F.Cu") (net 7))
 (segment (start 147.775 71.275) (end 148.5 72) (width 0.25) (layer "F.Cu") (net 7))
 (via (at 148.5 72) (size 1) (drill 0.6) (layers "F.Cu" "B.Cu") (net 7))
 (segment (start 148.5 73) (end 148 73) (width 0.25) (layer "B.Cu") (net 7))
 (segment (start 148.5 72) (end 148.5 73) (width 0.25) (layer "B.Cu") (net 7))
 (segment (start 146 75) (end 145.75 75) (width 0.25) (layer "B.Cu") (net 7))
 (segment (start 148 73) (end 146 75) (width 0.25) (layer "B.Cu") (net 7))
 (segment (start 148.875 70.625) (end 148.875 69.8725) (width 0.25) (layer "F.Cu") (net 8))
 (segment (start 149.5 71) (end 149.25 71) (width 0.25) (layer "F.Cu") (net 8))
 (segment (start 149.25 71) (end 148.875 70.625) (width 0.25) (layer "F.Cu") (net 8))
 (via (at 149.5 71) (size 1) (drill 0.6) (layers "F.Cu" "B.Cu") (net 8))
 (segment (start 151.25 72.5) (end 151 72.5) (width 0.25) (layer "B.Cu") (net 8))
 (segment (start 151 72.5) (end 149.5 71) (width 0.25) (layer "B.Cu") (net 8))
 (segment (start 135.1 76.47) (end 134.25 75.62) (width 0.25) (layer "B.Cu") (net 14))
 (segment (start 142.28 76.47) (end 135.1 76.47) (width 0.25) (layer "B.Cu") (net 14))
 (segment (start 143 75) (end 143 75.75) (width 0.25) (layer "B.Cu") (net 14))
 (segment (start 143 75.75) (end 142.28 76.47) (width 0.25) (layer "B.Cu") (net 14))
 (segment (start 148.5 75) (end 148.5 77) (width 0.25) (layer "B.Cu") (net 12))
 (segment (start 147.34 78.16) (end 134.25 78.16) (width 0.25) (layer "B.Cu") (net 12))
 (segment (start 148.5 77) (end 147.34 78.16) (width 0.25) (layer "B.Cu") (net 12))
 (segment (start 143.5 64.25) (end 136.75 64.25) (width 0.25) (layer "B.Cu") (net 10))
 (segment (start 134.21 65.21) (end 134.21 64.25) (width 0.25) (layer "B.Cu") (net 11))
 (segment (start 143 66) (end 142.75 65.75) (width 0.25) (layer "B.Cu") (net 11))
 (segment (start 134.75 65.75) (end 134.21 65.21) (width 0.25) (layer "B.Cu") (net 11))
 (segment (start 143 67) (end 143 66) (width 0.25) (layer "B.Cu") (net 11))
 (segment (start 142.75 65.75) (end 134.75 65.75) (width 0.25) (layer "B.Cu") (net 11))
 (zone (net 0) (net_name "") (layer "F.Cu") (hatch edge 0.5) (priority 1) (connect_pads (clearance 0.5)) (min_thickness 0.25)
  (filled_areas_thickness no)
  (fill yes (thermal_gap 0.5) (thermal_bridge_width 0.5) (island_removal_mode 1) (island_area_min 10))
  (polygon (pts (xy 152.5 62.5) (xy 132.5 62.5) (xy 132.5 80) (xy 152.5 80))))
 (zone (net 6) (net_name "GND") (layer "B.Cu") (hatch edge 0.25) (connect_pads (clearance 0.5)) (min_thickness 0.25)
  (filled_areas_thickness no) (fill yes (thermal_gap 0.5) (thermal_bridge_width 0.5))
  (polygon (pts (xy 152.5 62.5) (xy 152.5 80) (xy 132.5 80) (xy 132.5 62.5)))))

